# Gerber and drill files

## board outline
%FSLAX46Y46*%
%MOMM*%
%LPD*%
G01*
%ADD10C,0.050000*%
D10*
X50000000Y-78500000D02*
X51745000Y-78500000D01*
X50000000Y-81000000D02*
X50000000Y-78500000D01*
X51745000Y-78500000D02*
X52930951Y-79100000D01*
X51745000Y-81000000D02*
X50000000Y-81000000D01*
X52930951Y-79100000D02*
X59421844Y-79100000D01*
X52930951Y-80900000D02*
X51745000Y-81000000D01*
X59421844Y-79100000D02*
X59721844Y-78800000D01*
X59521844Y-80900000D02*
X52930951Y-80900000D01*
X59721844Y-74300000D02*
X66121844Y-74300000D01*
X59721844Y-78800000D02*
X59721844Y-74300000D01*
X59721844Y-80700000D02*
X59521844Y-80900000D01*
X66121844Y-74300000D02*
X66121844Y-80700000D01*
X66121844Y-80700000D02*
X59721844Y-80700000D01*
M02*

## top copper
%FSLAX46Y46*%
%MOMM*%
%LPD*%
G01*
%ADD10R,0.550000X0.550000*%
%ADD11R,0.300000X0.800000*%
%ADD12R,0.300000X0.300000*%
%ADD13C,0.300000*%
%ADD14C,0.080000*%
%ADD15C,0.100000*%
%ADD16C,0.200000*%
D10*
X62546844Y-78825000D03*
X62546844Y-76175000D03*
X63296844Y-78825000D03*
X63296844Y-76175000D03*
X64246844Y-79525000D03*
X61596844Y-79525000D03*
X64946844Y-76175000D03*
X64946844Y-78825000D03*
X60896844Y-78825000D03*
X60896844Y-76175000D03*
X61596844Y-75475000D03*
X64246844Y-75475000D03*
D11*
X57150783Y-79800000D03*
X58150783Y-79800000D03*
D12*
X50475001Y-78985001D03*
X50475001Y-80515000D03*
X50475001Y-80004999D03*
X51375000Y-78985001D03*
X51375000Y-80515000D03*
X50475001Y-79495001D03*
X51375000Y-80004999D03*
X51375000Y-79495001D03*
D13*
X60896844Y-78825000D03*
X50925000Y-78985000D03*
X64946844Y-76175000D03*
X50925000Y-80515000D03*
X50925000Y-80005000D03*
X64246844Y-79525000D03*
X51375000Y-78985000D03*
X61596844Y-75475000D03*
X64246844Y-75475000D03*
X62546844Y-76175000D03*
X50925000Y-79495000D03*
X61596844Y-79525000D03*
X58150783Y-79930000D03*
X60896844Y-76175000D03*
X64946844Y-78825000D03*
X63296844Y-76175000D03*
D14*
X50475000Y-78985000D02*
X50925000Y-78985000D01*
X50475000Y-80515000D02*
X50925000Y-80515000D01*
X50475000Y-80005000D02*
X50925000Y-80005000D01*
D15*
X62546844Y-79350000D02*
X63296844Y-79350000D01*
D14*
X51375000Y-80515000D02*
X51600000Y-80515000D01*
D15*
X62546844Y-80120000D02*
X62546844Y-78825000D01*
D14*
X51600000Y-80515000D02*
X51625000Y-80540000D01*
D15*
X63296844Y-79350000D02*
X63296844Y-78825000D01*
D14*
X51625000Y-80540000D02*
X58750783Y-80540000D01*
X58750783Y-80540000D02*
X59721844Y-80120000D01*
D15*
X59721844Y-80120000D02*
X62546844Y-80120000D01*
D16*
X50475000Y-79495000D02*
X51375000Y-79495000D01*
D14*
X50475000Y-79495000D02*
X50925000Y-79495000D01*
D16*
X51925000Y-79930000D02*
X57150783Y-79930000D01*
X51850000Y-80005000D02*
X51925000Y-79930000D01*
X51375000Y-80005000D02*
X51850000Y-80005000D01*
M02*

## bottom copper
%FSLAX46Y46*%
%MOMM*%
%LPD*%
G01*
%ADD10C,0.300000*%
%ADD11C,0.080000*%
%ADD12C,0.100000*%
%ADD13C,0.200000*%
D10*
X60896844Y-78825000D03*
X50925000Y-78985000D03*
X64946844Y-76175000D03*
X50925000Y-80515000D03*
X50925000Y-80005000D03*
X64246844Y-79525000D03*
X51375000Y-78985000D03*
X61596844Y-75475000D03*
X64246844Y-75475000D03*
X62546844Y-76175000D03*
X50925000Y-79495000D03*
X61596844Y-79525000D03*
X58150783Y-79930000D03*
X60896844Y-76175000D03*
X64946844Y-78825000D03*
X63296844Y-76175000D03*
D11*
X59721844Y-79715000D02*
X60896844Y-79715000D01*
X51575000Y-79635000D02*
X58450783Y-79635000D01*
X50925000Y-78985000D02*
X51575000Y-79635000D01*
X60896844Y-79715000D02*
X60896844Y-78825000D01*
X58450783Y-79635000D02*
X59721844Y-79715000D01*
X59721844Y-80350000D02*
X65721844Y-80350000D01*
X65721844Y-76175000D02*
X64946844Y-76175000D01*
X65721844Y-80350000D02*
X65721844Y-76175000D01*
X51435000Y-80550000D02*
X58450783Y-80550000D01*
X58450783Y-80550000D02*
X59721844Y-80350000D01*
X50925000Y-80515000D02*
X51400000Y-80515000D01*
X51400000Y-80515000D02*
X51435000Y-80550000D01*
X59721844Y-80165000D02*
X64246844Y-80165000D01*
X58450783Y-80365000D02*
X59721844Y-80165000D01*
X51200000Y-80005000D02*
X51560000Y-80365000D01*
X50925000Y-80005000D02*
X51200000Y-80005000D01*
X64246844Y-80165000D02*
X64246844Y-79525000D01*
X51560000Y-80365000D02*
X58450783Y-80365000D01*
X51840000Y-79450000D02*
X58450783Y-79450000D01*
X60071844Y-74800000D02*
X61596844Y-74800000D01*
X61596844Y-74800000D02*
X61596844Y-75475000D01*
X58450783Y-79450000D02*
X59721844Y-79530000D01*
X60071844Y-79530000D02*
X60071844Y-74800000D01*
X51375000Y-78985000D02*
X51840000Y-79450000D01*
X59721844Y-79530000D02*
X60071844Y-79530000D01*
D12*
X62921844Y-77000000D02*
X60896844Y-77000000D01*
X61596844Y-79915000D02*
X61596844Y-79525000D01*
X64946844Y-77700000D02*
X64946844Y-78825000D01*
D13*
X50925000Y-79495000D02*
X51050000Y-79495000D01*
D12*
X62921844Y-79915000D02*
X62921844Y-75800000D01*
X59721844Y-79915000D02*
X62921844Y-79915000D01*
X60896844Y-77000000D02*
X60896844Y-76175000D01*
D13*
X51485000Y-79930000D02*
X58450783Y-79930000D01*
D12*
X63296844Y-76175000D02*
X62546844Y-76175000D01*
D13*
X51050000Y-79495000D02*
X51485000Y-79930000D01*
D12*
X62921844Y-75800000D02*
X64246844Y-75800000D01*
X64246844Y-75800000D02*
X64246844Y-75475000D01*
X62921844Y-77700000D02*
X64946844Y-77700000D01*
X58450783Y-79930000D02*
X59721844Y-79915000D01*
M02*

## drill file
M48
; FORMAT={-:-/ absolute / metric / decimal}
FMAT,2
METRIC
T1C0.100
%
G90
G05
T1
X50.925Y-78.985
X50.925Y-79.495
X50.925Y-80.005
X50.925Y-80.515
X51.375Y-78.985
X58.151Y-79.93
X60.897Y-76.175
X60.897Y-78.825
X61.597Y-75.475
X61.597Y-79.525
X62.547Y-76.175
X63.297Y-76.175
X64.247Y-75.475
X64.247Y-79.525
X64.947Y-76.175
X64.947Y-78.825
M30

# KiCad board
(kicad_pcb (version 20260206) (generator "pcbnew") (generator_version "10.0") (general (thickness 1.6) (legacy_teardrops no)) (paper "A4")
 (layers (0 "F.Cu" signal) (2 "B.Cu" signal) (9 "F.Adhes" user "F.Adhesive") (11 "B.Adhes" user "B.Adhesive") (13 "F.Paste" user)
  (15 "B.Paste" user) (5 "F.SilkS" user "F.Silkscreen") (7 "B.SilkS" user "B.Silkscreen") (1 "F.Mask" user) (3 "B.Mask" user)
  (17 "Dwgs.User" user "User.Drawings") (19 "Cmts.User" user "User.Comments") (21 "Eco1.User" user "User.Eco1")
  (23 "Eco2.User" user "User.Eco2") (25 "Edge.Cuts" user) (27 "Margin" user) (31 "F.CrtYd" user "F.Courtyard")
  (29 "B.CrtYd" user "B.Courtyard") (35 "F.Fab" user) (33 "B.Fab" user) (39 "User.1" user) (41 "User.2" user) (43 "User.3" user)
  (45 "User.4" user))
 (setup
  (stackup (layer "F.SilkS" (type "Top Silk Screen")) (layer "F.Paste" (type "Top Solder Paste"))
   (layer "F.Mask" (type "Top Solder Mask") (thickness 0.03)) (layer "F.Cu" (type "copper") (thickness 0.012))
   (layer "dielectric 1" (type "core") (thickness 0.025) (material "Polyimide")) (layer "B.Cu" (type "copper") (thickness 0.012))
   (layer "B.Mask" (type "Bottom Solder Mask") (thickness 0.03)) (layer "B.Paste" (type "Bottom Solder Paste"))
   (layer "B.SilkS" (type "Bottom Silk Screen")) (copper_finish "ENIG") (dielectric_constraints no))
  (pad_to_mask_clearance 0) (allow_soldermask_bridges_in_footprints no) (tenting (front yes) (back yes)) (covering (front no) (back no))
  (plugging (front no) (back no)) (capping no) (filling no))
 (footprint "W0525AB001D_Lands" (layer "F.Cu") (at 57.650783 79.93)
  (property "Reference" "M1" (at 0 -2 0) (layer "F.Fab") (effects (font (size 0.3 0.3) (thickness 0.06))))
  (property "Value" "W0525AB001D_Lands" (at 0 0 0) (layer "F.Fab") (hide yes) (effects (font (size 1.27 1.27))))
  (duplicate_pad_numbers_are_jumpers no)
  (pad "1" smd rect (at -0.5 -0.13) (size 0.3 0.8) (layers "F.Cu" "F.Mask") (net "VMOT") (solder_mask_margin 0.05) (thermal_bridge_angle 45))
  (pad "2" smd rect (at 0.5 -0.13) (size 0.3 0.8) (layers "F.Cu" "F.Mask") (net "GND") (solder_mask_margin 0.05) (thermal_bridge_angle 45)))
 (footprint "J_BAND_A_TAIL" (layer "F.Cu") (at 50.9 79.75)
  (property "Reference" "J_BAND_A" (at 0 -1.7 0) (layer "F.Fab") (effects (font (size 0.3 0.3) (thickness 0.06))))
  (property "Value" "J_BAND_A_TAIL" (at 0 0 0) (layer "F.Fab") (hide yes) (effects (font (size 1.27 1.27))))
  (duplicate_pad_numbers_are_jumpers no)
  (pad "1" smd rect (at -0.424999 -0.764999) (size 0.3 0.3) (layers "F.Cu" "F.Mask") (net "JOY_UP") (solder_mask_margin 0.05)
   (thermal_bridge_angle 45))
  (pad "2" smd rect (at -0.424999 0.765) (size 0.3 0.3) (layers "F.Cu" "F.Mask") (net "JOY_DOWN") (solder_mask_margin 0.05)
   (thermal_bridge_angle 45))
  (pad "3" smd rect (at -0.424999 0.254999) (size 0.3 0.3) (layers "F.Cu" "F.Mask") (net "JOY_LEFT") (solder_mask_margin 0.05)
   (thermal_bridge_angle 45))
  (pad "4" smd rect (at 0.475 -0.764999) (size 0.3 0.3) (layers "F.Cu" "F.Mask") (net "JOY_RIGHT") (solder_mask_margin 0.05)
   (thermal_bridge_angle 45))
  (pad "5" smd rect (at 0.475 0.765) (size 0.3 0.3) (layers "F.Cu" "F.Mask") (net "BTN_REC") (solder_mask_margin 0.05)
   (thermal_bridge_angle 45))
  (pad "6" smd rect (at -0.424999 -0.254999) (size 0.3 0.3) (layers "F.Cu" "F.Mask") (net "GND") (solder_mask_margin 0.05)
   (thermal_bridge_angle 45))
  (pad "7" smd rect (at 0.475 0.254999) (size 0.3 0.3) (layers "F.Cu" "F.Mask") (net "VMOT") (solder_mask_margin 0.05)
   (thermal_bridge_angle 45))
  (pad "8" smd rect (at 0.475 -0.254999) (size 0.3 0.3) (layers "F.Cu" "F.Mask") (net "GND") (solder_mask_margin 0.05)
   (thermal_bridge_angle 45)))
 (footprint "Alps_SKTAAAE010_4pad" (layer "F.Cu") (at 62.921844 77.5 90)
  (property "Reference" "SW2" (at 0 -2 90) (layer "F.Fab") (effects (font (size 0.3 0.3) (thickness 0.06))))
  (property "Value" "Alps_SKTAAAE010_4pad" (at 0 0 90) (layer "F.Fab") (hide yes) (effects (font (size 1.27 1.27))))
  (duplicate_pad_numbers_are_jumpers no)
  (pad "1" smd rect (at -1.325 -0.375 90) (size 0.55 0.55) (layers "F.Cu" "F.Mask" "F.Paste") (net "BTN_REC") (solder_mask_margin 0.05)
   (thermal_bridge_angle 45))
  (pad "2" smd rect (at 1.325 -0.375 90) (size 0.55 0.55) (layers "F.Cu" "F.Mask" "F.Paste") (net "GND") (solder_mask_margin 0.05)
   (thermal_bridge_angle 45))
  (pad "3" smd rect (at -1.325 0.375 90) (size 0.55 0.55) (layers "F.Cu" "F.Mask" "F.Paste") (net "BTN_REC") (solder_mask_margin 0.05)
   (thermal_bridge_angle 45))
  (pad "4" smd rect (at 1.325 0.375 90) (size 0.55 0.55) (layers "F.Cu" "F.Mask" "F.Paste") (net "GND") (solder_mask_margin 0.05)
   (thermal_bridge_angle 45)))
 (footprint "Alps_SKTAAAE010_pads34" (layer "F.Cu") (at 62.921844 75.1)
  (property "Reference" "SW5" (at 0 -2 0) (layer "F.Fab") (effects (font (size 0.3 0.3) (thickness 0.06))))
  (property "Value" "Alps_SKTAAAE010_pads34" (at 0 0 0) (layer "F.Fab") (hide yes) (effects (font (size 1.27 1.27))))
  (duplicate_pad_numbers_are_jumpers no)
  (pad "3" smd rect (at -1.325 0.375) (size 0.55 0.55) (layers "F.Cu" "F.Mask" "F.Paste") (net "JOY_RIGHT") (solder_mask_margin 0.05)
   (thermal_bridge_angle 45))
  (pad "4" smd rect (at 1.325 0.375) (size 0.55 0.55) (layers "F.Cu" "F.Mask" "F.Paste") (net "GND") (solder_mask_margin 0.05)
   (thermal_bridge_angle 45)))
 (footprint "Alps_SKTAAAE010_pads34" (layer "F.Cu") (at 65.321844 77.5 -90)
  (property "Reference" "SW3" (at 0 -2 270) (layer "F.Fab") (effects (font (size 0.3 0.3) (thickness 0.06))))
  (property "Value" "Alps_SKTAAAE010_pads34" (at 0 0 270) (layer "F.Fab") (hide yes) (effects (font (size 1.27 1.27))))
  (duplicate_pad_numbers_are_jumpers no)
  (pad "3" smd rect (at -1.325 0.375 270) (size 0.55 0.55) (layers "F.Cu" "F.Mask" "F.Paste") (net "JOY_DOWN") (solder_mask_margin 0.05)
   (thermal_bridge_angle 45))
  (pad "4" smd rect (at 1.325 0.375 270) (size 0.55 0.55) (layers "F.Cu" "F.Mask" "F.Paste") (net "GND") (solder_mask_margin 0.05)
   (thermal_bridge_angle 45)))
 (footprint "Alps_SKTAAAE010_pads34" (layer "F.Cu") (at 62.921844 79.9 180)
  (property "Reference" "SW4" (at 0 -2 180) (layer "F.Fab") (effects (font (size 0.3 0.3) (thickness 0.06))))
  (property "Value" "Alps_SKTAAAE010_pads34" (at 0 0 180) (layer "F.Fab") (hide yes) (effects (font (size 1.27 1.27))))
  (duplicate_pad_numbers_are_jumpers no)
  (pad "3" smd rect (at -1.325 0.375 180) (size 0.55 0.55) (layers "F.Cu" "F.Mask" "F.Paste") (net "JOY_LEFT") (solder_mask_margin 0.05)
   (thermal_bridge_angle 45))
  (pad "4" smd rect (at 1.325 0.375 180) (size 0.55 0.55) (layers "F.Cu" "F.Mask" "F.Paste") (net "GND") (solder_mask_margin 0.05)
   (thermal_bridge_angle 45)))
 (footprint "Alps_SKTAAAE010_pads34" (layer "F.Cu") (at 60.521844 77.5 90)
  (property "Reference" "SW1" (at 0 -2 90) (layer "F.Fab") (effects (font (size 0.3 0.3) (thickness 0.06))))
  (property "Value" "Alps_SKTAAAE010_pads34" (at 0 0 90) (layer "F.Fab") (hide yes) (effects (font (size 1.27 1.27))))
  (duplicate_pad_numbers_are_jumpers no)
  (pad "3" smd rect (at -1.325 0.375 90) (size 0.55 0.55) (layers "F.Cu" "F.Mask" "F.Paste") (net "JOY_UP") (solder_mask_margin 0.05)
   (thermal_bridge_angle 45))
  (pad "4" smd rect (at 1.325 0.375 90) (size 0.55 0.55) (layers "F.Cu" "F.Mask" "F.Paste") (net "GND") (solder_mask_margin 0.05)
   (thermal_bridge_angle 45)))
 (gr_line (start 50 78.5) (end 51.745 78.5) (stroke (width 0.05) (type default)) (layer "Edge.Cuts"))
 (gr_line (start 50 81) (end 50 78.5) (stroke (width 0.05) (type default)) (layer "Edge.Cuts"))
 (gr_line (start 51.745 78.5) (end 52.930951 79.1) (stroke (width 0.05) (type default)) (layer "Edge.Cuts"))
 (gr_line (start 51.745 81) (end 50 81) (stroke (width 0.05) (type default)) (layer "Edge.Cuts"))
 (gr_line (start 52.930951 79.1) (end 59.421844 79.1) (stroke (width 0.05) (type default)) (layer "Edge.Cuts"))
 (gr_line (start 52.930951 80.9) (end 51.745 81) (stroke (width 0.05) (type default)) (layer "Edge.Cuts"))
 (gr_line (start 59.421844 79.1) (end 59.721844 78.8) (stroke (width 0.05) (type default)) (layer "Edge.Cuts"))
 (gr_line (start 59.521844 80.9) (end 52.930951 80.9) (stroke (width 0.05) (type default)) (layer "Edge.Cuts"))
 (gr_line (start 59.721844 74.3) (end 66.121844 74.3) (stroke (width 0.05) (type default)) (layer "Edge.Cuts"))
 (gr_line (start 59.721844 78.8) (end 59.721844 74.3) (stroke (width 0.05) (type default)) (layer "Edge.Cuts"))
 (gr_line (start 59.721844 80.7) (end 59.521844 80.9) (stroke (width 0.05) (type default)) (layer "Edge.Cuts"))
 (gr_line (start 66.121844 74.3) (end 66.121844 80.7) (stroke (width 0.05) (type default)) (layer "Edge.Cuts"))
 (gr_line (start 66.121844 80.7) (end 59.721844 80.7) (stroke (width 0.05) (type default)) (layer "Edge.Cuts"))
 (segment (start 50.475 78.985) (end 50.925 78.985) (width 0.08) (layer "F.Cu") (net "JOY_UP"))
 (via (at 60.896844 78.825) (size 0.3) (drill 0.1) (layers "F.Cu" "B.Cu") (tenting (front yes) (back yes)) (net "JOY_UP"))
 (via (at 50.925 78.985) (size 0.3) (drill 0.1) (layers "F.Cu" "B.Cu") (tenting (front yes) (back yes)) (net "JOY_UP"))
 (segment (start 51.575 79.635) (end 58.450783 79.635) (width 0.08) (layer "B.Cu") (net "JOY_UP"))
 (segment (start 60.896844 79.715) (end 60.896844 78.825) (width 0.08) (layer "B.Cu") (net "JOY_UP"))
 (segment (start 59.721844 79.715) (end 60.896844 79.715) (width 0.08) (layer "B.Cu") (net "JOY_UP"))
 (segment (start 50.925 78.985) (end 51.575 79.635) (width 0.08) (layer "B.Cu") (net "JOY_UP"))
 (segment (start 58.450783 79.635) (end 59.721844 79.715) (width 0.08) (layer "B.Cu") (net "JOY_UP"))
 (segment (start 50.475 80.515) (end 50.925 80.515) (width 0.08) (layer "F.Cu") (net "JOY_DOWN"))
 (via (at 50.925 80.515) (size 0.3) (drill 0.1) (layers "F.Cu" "B.Cu") (tenting (front yes) (back yes)) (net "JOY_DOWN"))
 (via (at 64.946844 76.175) (size 0.3) (drill 0.1) (layers "F.Cu" "B.Cu") (tenting (front yes) (back yes)) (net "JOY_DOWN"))
 (segment (start 59.721844 80.35) (end 65.721844 80.35) (width 0.08) (layer "B.Cu") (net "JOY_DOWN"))
 (segment (start 65.721844 80.35) (end 65.721844 76.175) (width 0.08) (layer "B.Cu") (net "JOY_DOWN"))
 (segment (start 51.4 80.515) (end 51.435 80.55) (width 0.08) (layer "B.Cu") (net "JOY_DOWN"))
 (segment (start 65.721844 76.175) (end 64.946844 76.175) (width 0.08) (layer "B.Cu") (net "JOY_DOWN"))
 (segment (start 50.925 80.515) (end 51.4 80.515) (width 0.08) (layer "B.Cu") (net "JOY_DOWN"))
 (segment (start 58.450783 80.55) (end 59.721844 80.35) (width 0.08) (layer "B.Cu") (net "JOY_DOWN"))
 (segment (start 51.435 80.55) (end 58.450783 80.55) (width 0.08) (layer "B.Cu") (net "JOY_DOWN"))
 (segment (start 50.475 80.005) (end 50.925 80.005) (width 0.08) (layer "F.Cu") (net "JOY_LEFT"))
 (via (at 50.925 80.005) (size 0.3) (drill 0.1) (layers "F.Cu" "B.Cu") (tenting (front yes) (back yes)) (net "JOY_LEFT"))
 (via (at 64.246844 79.525) (size 0.3) (drill 0.1) (layers "F.Cu" "B.Cu") (tenting (front yes) (back yes)) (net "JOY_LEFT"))
 (segment (start 51.2 80.005) (end 51.56 80.365) (width 0.08) (layer "B.Cu") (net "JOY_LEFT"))
 (segment (start 51.56 80.365) (end 58.450783 80.365) (width 0.08) (layer "B.Cu") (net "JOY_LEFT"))
 (segment (start 59.721844 80.165) (end 64.246844 80.165) (width 0.08) (layer "B.Cu") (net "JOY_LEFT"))
 (segment (start 50.925 80.005) (end 51.2 80.005) (width 0.08) (layer "B.Cu") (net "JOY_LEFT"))
 (segment (start 58.450783 80.365) (end 59.721844 80.165) (width 0.08) (layer "B.Cu") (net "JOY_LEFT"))
 (segment (start 64.246844 80.165) (end 64.246844 79.525) (width 0.08) (layer "B.Cu") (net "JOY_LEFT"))
 (via (at 61.596844 75.475) (size 0.3) (drill 0.1) (layers "F.Cu" "B.Cu") (tenting (front yes) (back yes)) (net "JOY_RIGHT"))
 (via (at 51.375 78.985) (size 0.3) (drill 0.1) (layers "F.Cu" "B.Cu") (tenting (front yes) (back yes)) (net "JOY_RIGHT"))
 (segment (start 60.071844 79.53) (end 60.071844 74.8) (width 0.08) (layer "B.Cu") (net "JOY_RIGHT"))
 (segment (start 58.450783 79.45) (end 59.721844 79.53) (width 0.08) (layer "B.Cu") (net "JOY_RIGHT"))
 (segment (start 59.721844 79.53) (end 60.071844 79.53) (width 0.08) (layer "B.Cu") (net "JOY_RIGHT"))
 (segment (start 51.84 79.45) (end 58.450783 79.45) (width 0.08) (layer "B.Cu") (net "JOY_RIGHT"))
 (segment (start 60.071844 74.8) (end 61.596844 74.8) (width 0.08) (layer "B.Cu") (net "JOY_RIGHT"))
 (segment (start 61.596844 74.8) (end 61.596844 75.475) (width 0.08) (layer "B.Cu") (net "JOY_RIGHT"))
 (segment (start 51.375 78.985) (end 51.84 79.45) (width 0.08) (layer "B.Cu") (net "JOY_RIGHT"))
 (segment (start 62.546844 79.35) (end 63.296844 79.35) (width 0.1) (layer "F.Cu") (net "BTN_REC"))
 (segment (start 62.546844 80.12) (end 62.546844 78.825) (width 0.1) (layer "F.Cu") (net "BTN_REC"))
 (segment (start 51.625 80.54) (end 58.750783 80.54) (width 0.08) (layer "F.Cu") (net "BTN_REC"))
 (segment (start 59.721844 80.12) (end 62.546844 80.12) (width 0.1) (layer "F.Cu") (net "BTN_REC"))
 (segment (start 58.750783 80.54) (end 59.721844 80.12) (width 0.08) (layer "F.Cu") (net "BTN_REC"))
 (segment (start 51.6 80.515) (end 51.625 80.54) (width 0.08) (layer "F.Cu") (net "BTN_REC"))
 (segment (start 63.296844 79.35) (end 63.296844 78.825) (width 0.1) (layer "F.Cu") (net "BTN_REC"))
 (segment (start 51.375 80.515) (end 51.6 80.515) (width 0.08) (layer "F.Cu") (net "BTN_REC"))
 (segment (start 50.475 79.495) (end 50.925 79.495) (width 0.08) (layer "F.Cu") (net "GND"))
 (segment (start 50.475 79.495) (end 51.375 79.495) (width 0.2) (layer "F.Cu") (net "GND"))
 (via (at 63.296844 76.175) (size 0.3) (drill 0.1) (layers "F.Cu" "B.Cu") (tenting (front yes) (back yes)) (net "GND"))
 (via (at 62.546844 76.175) (size 0.3) (drill 0.1) (layers "F.Cu" "B.Cu") (tenting (front yes) (back yes)) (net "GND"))
 (via (at 58.150783 79.93) (size 0.3) (drill 0.1) (layers "F.Cu" "B.Cu") (tenting (front yes) (back yes)) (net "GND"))
 (via (at 60.896844 76.175) (size 0.3) (drill 0.1) (layers "F.Cu" "B.Cu") (tenting (front yes) (back yes)) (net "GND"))
 (via (at 64.946844 78.825) (size 0.3) (drill 0.1) (layers "F.Cu" "B.Cu") (tenting (front yes) (back yes)) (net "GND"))
 (via (at 64.246844 75.475) (size 0.3) (drill 0.1) (layers "F.Cu" "B.Cu") (tenting (front yes) (back yes)) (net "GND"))
 (via (at 50.925 79.495) (size 0.3) (drill 0.1) (layers "F.Cu" "B.Cu") (tenting (front yes) (back yes)) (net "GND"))
 (via (at 61.596844 79.525) (size 0.3) (drill 0.1) (layers "F.Cu" "B.Cu") (tenting (front yes) (back yes)) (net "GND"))
 (segment (start 64.946844 77.7) (end 64.946844 78.825) (width 0.1) (layer "B.Cu") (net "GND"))
 (segment (start 64.246844 75.8) (end 64.246844 75.475) (width 0.1) (layer "B.Cu") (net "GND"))
 (segment (start 51.485 79.93) (end 58.450783 79.93) (width 0.2) (layer "B.Cu") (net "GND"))
 (segment (start 58.450783 79.93) (end 59.721844 79.915) (width 0.1) (layer "B.Cu") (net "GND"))
 (segment (start 59.721844 79.915) (end 62.921844 79.915) (width 0.1) (layer "B.Cu") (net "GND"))
 (segment (start 62.921844 75.8) (end 64.246844 75.8) (width 0.1) (layer "B.Cu") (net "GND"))
 (segment (start 50.925 79.495) (end 51.05 79.495) (width 0.2) (layer "B.Cu") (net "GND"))
 (segment (start 51.05 79.495) (end 51.485 79.93) (width 0.2) (layer "B.Cu") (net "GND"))
 (segment (start 62.921844 77.7) (end 64.946844 77.7) (width 0.1) (layer "B.Cu") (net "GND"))
 (segment (start 61.596844 79.915) (end 61.596844 79.525) (width 0.1) (layer "B.Cu") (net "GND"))
 (segment (start 63.296844 76.175) (end 62.546844 76.175) (width 0.1) (layer "B.Cu") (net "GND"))
 (segment (start 60.896844 77) (end 60.896844 76.175) (width 0.1) (layer "B.Cu") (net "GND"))
 (segment (start 62.921844 77) (end 60.896844 77) (width 0.1) (layer "B.Cu") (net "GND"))
 (segment (start 62.921844 79.915) (end 62.921844 75.8) (width 0.1) (layer "B.Cu") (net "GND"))
 (segment (start 51.925 79.93) (end 57.150783 79.93) (width 0.2) (layer "F.Cu") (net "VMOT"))
 (segment (start 51.85 80.005) (end 51.925 79.93) (width 0.2) (layer "F.Cu") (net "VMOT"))
 (segment (start 51.375 80.005) (end 51.85 80.005) (width 0.2) (layer "F.Cu") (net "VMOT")))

